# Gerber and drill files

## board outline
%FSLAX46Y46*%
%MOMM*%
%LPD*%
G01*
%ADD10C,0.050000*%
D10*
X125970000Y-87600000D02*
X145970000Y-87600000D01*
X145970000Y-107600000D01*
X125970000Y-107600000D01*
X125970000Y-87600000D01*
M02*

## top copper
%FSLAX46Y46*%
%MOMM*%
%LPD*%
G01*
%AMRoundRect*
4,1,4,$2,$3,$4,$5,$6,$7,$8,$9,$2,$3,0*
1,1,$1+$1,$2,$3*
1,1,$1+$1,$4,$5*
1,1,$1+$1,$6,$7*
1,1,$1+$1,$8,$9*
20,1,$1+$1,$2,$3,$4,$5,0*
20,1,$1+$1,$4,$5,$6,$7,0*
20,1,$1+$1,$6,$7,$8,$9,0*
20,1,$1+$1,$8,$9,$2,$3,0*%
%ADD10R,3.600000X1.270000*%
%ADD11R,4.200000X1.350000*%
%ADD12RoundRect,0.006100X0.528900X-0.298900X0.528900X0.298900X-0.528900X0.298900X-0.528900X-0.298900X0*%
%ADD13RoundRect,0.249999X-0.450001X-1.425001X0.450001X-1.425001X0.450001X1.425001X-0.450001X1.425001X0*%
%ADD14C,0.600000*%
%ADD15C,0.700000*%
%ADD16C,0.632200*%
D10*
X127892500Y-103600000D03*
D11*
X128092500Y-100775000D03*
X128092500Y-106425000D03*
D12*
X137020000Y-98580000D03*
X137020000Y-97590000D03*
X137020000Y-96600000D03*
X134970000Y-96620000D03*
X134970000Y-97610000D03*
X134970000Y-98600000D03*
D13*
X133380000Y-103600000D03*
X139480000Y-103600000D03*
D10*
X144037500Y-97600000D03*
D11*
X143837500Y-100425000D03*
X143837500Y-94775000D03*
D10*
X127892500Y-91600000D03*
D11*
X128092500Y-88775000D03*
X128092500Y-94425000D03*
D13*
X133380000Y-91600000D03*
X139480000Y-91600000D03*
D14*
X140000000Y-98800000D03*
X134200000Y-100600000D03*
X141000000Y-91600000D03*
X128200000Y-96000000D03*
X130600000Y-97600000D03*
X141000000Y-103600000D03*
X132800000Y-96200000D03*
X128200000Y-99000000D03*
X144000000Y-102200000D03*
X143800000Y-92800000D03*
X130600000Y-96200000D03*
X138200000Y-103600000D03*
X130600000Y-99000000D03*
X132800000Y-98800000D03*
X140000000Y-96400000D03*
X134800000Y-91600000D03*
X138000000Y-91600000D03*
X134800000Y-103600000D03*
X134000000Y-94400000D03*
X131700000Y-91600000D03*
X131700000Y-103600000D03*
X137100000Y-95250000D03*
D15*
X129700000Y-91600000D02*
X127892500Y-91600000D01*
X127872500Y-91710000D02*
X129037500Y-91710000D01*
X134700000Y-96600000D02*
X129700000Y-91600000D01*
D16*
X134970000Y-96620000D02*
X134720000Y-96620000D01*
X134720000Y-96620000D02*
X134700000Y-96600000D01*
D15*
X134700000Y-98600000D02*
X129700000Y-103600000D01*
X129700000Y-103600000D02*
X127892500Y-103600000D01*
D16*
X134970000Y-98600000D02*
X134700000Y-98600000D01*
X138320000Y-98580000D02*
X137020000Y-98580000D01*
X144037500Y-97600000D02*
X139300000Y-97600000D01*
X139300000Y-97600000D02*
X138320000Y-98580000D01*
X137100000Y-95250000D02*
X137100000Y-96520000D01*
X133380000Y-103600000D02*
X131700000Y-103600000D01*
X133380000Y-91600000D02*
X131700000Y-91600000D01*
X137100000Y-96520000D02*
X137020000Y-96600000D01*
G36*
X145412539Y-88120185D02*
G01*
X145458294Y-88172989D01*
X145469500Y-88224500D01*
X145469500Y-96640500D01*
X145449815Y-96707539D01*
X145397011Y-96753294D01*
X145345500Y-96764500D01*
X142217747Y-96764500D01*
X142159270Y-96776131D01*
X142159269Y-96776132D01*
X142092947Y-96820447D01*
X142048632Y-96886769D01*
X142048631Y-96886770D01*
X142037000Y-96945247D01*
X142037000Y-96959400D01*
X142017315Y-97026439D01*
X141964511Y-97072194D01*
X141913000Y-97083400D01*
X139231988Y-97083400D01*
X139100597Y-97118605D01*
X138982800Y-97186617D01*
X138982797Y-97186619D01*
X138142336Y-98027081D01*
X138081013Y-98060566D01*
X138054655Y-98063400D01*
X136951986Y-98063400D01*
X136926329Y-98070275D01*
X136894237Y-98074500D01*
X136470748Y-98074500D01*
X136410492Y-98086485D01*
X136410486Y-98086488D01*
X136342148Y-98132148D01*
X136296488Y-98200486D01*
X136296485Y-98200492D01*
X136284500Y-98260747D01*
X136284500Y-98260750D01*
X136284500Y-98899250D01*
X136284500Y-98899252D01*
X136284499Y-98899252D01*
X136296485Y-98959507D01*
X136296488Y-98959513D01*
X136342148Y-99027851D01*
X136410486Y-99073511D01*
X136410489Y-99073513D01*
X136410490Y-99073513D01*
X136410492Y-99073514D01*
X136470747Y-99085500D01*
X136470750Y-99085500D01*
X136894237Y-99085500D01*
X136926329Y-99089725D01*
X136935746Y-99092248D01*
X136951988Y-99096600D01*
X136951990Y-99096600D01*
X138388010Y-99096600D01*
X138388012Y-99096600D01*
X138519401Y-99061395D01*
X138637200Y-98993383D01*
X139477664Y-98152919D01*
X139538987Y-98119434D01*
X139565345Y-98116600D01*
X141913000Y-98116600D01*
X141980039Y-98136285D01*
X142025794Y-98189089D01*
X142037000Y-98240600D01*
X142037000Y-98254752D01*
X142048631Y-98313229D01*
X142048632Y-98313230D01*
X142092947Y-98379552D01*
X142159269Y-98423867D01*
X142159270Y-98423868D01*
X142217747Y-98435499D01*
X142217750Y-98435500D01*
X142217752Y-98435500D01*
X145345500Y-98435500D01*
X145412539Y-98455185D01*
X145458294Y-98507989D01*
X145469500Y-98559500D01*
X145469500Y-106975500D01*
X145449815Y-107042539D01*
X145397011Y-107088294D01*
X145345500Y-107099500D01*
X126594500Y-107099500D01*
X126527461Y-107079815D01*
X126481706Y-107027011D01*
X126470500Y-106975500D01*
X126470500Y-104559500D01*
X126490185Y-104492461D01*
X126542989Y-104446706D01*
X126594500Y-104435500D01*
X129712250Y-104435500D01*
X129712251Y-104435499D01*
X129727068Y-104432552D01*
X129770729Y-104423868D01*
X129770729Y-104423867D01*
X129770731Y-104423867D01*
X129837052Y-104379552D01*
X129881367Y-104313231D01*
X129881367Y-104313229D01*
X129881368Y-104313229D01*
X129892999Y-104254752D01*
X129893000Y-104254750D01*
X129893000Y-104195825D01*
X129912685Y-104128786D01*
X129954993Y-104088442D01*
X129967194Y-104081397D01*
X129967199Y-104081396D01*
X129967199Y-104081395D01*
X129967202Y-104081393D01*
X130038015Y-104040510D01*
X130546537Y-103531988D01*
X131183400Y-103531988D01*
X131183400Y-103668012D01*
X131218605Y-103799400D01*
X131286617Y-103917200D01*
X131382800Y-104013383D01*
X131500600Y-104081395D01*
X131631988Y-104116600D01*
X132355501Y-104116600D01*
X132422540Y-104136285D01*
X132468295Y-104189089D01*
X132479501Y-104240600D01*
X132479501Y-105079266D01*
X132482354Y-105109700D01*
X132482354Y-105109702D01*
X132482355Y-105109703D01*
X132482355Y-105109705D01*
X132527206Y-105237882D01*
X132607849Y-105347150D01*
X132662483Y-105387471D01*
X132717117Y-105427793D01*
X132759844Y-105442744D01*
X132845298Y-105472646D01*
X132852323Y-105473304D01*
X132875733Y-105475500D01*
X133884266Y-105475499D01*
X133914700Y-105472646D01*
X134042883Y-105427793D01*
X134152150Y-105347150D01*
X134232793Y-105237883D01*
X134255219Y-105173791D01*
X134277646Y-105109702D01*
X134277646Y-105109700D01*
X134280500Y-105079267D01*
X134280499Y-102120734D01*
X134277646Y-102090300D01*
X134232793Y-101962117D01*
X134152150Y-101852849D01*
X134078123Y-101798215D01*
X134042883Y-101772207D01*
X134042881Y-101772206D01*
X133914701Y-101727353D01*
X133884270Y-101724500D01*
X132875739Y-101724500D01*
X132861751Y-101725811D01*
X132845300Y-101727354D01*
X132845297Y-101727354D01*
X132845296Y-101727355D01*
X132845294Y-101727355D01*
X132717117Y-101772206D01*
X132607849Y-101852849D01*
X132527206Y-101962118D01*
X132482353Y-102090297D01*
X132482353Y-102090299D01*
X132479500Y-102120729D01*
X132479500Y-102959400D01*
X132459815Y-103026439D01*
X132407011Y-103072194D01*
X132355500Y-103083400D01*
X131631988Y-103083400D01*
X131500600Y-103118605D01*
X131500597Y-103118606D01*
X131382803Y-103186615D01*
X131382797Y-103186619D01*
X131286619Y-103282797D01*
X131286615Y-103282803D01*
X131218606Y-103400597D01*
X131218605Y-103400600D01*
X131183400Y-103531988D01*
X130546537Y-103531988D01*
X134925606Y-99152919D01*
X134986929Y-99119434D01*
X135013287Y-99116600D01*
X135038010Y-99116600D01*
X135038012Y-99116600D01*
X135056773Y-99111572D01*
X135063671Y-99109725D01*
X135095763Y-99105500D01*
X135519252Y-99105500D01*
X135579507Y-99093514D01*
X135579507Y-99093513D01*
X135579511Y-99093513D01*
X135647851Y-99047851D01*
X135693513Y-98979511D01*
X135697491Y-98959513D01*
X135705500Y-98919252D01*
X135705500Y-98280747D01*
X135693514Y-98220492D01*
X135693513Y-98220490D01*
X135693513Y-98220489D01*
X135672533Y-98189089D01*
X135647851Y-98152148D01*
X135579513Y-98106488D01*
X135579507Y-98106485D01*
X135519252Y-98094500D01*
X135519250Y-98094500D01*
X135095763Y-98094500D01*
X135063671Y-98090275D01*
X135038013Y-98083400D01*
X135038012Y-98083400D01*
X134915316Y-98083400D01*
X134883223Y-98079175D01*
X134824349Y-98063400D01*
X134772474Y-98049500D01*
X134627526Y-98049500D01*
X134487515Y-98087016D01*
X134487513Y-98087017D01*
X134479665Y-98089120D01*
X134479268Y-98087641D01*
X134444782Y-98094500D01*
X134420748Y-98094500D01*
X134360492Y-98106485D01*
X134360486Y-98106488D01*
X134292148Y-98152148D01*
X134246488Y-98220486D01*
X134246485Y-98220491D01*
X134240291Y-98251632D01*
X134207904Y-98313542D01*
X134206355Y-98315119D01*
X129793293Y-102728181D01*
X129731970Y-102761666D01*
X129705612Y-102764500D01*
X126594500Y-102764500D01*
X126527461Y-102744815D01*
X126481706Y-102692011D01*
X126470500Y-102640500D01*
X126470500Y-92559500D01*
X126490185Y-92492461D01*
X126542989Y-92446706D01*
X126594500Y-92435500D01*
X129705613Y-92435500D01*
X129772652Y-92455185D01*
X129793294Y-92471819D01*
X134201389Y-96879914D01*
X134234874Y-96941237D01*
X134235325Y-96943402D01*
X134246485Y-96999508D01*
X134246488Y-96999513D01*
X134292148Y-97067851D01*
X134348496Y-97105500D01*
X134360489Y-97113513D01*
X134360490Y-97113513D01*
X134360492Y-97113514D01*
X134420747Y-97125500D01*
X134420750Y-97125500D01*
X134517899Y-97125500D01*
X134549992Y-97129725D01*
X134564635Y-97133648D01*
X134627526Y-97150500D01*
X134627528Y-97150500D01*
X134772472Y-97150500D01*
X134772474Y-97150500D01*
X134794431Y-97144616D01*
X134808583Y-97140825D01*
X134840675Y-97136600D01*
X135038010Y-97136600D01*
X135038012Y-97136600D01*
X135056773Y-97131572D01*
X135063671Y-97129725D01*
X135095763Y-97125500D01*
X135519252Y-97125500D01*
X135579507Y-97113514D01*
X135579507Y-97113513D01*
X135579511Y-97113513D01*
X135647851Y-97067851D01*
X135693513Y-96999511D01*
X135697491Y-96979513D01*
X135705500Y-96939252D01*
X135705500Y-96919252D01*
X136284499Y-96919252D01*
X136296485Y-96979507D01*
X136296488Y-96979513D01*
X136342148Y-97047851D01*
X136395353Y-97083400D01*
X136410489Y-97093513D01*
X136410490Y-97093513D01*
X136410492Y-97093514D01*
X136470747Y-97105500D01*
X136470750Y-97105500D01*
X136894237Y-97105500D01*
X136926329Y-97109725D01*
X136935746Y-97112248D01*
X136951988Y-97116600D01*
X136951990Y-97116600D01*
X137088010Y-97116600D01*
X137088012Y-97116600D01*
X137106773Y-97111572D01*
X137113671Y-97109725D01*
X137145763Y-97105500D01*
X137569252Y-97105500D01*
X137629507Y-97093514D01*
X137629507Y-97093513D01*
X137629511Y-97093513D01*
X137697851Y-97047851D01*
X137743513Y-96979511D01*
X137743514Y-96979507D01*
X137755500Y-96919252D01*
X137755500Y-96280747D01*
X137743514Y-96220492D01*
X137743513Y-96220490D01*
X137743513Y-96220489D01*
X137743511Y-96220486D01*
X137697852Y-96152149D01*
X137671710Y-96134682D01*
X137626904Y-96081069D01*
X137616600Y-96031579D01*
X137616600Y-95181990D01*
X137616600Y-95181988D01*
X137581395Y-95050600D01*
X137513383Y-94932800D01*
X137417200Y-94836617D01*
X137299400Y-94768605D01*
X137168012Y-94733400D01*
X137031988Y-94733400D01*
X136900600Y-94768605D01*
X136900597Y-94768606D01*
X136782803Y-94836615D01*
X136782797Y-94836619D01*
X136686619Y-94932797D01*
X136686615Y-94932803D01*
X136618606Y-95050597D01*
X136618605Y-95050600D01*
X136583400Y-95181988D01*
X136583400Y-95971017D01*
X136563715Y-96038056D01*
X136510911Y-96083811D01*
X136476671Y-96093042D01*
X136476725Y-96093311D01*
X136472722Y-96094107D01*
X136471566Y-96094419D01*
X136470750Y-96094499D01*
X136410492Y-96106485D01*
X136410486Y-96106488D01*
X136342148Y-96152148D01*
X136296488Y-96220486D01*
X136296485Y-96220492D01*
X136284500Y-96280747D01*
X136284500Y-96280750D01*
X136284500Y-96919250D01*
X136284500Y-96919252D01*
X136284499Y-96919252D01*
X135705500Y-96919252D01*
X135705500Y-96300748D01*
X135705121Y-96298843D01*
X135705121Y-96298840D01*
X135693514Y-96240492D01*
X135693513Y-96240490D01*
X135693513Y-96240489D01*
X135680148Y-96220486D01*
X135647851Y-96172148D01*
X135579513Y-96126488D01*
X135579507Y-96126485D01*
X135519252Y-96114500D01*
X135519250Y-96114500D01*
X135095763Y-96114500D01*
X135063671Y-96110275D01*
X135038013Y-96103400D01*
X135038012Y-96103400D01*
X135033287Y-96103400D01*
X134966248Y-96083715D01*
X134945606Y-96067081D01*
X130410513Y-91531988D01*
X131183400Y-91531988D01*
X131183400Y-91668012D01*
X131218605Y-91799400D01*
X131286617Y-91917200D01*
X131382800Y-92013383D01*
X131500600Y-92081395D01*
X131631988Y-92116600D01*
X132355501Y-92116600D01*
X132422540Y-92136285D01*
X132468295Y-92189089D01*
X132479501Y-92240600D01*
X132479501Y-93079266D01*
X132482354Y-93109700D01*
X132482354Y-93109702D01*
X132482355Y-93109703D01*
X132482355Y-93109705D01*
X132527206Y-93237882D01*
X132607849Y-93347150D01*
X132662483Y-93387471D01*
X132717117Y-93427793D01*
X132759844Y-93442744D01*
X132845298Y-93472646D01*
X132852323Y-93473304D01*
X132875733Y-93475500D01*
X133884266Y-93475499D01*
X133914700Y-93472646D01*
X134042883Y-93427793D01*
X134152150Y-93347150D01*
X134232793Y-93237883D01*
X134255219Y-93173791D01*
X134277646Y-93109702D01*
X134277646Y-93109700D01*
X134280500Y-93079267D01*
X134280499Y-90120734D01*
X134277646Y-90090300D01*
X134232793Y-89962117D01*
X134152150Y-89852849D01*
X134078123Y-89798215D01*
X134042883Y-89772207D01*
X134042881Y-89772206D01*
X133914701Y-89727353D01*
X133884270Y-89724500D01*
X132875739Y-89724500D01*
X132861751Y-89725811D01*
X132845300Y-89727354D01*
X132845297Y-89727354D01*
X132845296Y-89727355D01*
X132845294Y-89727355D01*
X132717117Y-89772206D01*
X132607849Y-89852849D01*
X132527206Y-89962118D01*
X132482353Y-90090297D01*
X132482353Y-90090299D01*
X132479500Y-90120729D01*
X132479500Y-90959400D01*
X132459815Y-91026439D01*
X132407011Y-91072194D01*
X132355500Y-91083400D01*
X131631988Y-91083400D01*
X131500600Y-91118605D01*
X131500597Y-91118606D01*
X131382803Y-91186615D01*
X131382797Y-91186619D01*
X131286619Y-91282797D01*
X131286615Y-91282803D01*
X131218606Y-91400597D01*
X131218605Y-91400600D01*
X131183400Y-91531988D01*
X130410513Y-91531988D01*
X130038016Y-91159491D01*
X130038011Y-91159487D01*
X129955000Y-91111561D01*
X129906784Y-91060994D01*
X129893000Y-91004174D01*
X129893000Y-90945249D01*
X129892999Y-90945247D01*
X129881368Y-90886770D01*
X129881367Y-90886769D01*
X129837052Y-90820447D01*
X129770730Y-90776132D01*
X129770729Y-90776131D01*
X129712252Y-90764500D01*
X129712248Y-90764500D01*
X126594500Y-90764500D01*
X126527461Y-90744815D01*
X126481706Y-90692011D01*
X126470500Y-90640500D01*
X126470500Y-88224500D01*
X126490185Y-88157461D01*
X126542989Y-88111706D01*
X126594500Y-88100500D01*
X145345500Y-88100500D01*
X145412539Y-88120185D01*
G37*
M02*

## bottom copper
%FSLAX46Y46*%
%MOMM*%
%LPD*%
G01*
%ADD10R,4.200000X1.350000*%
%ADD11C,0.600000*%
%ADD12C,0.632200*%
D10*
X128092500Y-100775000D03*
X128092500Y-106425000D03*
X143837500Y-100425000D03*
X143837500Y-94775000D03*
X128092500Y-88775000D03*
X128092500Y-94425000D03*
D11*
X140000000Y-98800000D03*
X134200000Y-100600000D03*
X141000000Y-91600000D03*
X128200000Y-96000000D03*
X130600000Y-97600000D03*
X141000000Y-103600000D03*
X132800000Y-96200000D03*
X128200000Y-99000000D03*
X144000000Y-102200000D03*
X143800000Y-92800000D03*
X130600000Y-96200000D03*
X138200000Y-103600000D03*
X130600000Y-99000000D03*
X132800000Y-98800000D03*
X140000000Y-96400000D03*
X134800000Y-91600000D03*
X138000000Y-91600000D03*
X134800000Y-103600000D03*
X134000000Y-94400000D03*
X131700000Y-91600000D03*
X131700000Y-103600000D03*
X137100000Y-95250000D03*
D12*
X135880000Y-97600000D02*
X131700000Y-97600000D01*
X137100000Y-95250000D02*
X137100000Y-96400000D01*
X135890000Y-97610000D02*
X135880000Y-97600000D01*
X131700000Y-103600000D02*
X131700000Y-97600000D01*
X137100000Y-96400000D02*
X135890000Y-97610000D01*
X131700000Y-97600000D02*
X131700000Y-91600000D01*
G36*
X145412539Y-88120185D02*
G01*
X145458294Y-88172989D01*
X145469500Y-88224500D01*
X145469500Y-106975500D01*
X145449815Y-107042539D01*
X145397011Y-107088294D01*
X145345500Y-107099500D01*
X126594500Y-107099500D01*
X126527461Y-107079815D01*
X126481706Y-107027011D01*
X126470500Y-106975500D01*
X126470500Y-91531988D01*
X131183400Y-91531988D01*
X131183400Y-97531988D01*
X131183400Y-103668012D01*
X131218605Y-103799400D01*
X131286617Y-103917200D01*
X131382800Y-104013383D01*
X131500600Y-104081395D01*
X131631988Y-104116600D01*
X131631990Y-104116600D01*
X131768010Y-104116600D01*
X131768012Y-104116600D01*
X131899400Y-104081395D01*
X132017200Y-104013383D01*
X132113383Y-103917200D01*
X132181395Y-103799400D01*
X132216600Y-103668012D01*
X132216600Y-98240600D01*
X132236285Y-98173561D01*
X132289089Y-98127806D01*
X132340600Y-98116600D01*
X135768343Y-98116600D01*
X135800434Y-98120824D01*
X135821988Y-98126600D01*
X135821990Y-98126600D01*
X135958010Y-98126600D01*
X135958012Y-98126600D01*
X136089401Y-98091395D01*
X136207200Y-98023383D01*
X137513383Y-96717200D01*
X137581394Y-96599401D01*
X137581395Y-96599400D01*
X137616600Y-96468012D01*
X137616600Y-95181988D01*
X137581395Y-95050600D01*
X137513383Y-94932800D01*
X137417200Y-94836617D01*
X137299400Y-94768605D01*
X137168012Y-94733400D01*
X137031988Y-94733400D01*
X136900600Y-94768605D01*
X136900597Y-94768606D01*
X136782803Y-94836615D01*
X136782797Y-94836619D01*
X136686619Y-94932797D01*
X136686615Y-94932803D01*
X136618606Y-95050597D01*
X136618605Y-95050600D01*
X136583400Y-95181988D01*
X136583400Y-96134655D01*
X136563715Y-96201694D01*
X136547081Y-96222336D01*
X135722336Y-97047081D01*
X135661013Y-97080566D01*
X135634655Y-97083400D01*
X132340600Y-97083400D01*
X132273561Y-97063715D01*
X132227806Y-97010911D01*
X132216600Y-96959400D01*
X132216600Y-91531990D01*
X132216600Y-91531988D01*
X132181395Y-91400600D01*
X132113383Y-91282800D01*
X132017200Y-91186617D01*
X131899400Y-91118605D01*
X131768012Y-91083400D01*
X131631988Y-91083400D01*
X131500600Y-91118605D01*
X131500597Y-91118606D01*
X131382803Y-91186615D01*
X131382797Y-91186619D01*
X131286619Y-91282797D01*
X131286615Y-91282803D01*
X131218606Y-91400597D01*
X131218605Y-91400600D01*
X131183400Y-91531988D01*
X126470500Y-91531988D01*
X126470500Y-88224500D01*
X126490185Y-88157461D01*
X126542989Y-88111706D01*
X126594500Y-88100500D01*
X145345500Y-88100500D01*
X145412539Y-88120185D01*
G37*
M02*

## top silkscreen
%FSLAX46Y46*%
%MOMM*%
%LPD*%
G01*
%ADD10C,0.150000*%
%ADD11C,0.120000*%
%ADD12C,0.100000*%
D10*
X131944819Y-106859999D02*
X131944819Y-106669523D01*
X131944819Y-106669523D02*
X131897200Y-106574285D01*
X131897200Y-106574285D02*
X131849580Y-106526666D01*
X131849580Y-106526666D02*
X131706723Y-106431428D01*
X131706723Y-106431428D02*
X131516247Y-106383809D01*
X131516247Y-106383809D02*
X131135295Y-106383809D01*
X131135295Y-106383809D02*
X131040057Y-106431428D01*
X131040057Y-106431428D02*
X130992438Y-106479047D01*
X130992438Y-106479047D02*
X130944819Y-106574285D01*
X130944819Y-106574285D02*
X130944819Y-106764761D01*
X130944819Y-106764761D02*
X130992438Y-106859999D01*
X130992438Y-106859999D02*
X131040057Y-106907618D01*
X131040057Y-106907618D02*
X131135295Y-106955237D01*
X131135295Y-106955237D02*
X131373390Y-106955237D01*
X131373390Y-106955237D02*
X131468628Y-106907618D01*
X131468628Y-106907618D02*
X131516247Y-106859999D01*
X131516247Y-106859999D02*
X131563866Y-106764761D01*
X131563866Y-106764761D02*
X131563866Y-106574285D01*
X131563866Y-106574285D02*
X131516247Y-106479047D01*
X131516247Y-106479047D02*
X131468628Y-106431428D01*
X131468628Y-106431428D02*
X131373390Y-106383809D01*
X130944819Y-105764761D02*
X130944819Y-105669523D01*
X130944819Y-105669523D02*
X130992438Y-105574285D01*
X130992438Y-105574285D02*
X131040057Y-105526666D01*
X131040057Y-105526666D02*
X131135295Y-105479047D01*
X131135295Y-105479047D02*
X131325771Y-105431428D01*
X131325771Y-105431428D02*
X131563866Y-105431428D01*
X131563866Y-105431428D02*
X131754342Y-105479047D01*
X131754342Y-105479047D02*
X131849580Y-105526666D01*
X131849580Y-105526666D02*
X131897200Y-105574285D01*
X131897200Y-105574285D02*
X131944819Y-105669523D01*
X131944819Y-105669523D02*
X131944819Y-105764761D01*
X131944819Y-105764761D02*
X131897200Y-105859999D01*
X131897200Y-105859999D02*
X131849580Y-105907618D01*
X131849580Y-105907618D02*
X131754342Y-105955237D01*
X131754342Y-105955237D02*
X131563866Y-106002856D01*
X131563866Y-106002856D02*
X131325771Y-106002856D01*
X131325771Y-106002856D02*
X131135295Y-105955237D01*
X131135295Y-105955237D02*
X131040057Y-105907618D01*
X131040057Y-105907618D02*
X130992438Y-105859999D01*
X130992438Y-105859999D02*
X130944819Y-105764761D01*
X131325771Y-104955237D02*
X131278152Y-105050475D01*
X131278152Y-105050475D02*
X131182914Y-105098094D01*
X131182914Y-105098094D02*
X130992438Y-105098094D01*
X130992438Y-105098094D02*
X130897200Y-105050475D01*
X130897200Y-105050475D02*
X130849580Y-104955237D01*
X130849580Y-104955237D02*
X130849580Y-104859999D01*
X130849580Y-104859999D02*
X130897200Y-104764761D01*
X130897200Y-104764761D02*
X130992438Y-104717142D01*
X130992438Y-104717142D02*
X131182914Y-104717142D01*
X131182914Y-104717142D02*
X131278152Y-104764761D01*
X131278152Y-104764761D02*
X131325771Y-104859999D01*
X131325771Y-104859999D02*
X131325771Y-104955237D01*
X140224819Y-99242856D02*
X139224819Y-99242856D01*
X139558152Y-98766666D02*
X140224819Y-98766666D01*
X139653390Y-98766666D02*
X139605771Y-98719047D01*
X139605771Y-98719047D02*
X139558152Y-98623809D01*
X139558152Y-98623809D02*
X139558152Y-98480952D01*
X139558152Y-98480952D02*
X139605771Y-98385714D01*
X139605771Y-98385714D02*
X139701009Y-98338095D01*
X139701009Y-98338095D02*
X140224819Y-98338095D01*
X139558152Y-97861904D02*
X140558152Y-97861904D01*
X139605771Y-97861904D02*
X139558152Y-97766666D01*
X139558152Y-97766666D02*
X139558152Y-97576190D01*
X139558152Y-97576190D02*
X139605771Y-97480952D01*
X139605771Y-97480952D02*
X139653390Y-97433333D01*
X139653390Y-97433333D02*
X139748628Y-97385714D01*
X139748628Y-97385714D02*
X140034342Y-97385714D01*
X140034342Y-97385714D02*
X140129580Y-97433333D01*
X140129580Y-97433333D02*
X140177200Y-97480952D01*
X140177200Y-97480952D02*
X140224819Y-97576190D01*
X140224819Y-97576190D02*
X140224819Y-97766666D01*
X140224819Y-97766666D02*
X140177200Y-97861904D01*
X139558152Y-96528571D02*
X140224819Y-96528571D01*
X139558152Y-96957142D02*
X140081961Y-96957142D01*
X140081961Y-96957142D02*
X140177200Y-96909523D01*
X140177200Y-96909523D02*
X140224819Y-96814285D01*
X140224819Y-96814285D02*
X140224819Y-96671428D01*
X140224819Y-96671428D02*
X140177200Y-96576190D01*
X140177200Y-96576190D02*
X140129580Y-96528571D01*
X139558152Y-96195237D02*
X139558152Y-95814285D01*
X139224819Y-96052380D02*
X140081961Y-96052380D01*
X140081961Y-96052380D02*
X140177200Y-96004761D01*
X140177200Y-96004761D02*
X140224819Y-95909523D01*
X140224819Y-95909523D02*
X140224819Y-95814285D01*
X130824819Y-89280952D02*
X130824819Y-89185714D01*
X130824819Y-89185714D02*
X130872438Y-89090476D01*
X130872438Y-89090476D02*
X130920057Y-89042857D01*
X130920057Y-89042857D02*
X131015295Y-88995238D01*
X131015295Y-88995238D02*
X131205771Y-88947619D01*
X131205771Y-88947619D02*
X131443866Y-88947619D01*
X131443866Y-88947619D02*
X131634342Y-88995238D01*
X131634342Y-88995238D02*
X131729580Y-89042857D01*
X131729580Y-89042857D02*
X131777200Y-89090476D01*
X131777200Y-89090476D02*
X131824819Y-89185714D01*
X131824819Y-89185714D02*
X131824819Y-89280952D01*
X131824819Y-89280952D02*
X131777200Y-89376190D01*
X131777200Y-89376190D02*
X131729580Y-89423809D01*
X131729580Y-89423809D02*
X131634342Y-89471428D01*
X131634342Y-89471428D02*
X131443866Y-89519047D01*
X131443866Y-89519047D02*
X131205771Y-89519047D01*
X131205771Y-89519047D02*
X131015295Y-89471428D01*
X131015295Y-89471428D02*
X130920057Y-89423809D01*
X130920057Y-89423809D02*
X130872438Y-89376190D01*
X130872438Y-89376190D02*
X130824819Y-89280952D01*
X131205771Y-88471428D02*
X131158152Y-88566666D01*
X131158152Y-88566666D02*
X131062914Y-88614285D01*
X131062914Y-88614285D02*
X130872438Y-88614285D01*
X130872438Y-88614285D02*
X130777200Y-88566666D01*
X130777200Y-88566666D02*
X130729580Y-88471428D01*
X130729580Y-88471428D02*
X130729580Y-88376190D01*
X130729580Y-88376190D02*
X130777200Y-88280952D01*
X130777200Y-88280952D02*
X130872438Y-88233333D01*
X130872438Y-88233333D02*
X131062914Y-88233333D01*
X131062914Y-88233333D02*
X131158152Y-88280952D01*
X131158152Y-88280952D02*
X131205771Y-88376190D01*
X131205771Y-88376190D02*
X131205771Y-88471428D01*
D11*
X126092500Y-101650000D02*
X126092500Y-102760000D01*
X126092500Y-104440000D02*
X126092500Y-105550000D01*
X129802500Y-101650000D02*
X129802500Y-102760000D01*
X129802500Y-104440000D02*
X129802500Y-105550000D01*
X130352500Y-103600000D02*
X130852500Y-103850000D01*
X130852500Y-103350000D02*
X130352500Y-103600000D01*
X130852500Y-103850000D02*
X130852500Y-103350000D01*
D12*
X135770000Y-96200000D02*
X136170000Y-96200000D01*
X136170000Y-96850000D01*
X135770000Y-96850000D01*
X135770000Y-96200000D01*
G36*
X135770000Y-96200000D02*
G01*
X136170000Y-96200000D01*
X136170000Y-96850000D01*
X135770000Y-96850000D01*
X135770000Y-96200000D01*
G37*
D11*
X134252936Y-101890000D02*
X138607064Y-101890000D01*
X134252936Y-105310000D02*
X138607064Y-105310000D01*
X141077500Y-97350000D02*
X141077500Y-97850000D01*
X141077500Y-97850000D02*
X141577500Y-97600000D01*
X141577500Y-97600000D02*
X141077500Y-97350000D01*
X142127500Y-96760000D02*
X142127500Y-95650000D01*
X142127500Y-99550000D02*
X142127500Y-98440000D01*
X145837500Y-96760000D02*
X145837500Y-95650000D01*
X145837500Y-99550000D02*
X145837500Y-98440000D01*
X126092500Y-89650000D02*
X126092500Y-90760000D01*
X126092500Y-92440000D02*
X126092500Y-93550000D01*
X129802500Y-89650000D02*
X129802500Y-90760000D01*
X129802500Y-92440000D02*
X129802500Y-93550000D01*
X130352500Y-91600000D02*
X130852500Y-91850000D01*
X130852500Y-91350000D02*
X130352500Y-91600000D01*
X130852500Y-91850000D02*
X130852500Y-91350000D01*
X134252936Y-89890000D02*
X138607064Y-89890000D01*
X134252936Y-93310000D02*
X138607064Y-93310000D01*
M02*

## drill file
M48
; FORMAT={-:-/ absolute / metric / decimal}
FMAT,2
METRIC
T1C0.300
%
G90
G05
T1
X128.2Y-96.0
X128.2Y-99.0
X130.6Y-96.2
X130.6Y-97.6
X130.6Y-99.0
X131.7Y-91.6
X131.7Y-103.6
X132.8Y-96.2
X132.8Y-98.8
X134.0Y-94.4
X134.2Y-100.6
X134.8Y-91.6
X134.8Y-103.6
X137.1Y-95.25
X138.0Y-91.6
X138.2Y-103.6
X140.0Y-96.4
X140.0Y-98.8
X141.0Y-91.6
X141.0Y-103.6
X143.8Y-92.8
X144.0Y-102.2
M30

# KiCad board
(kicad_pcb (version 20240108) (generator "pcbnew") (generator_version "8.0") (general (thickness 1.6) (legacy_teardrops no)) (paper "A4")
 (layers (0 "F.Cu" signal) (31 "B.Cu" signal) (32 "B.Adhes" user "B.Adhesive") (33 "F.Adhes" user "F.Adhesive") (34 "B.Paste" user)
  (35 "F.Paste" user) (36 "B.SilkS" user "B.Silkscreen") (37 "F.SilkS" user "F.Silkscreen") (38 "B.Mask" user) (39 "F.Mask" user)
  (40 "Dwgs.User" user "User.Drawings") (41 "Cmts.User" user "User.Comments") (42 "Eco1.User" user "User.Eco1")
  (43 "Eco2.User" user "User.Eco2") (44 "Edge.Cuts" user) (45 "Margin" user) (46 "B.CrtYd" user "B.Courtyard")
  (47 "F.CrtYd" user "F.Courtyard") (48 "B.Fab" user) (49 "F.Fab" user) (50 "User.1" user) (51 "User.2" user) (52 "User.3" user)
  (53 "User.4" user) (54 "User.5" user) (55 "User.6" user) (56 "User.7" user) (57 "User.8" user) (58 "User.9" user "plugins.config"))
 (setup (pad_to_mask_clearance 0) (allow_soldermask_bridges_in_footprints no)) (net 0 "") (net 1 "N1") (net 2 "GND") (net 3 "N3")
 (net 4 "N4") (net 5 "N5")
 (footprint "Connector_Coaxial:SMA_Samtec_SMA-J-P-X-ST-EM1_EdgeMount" (layer "F.Cu") (at 128.0925 103.6 -90)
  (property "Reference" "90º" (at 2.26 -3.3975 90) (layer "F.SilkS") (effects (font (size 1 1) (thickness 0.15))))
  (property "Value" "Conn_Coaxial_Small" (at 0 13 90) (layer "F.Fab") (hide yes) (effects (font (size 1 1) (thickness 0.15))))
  (fp_line (start -1.95 2) (end -0.84 2) (stroke (width 0.12) (type solid)) (layer "F.SilkS"))
  (fp_line (start 0.84 2) (end 1.95 2) (stroke (width 0.12) (type solid)) (layer "F.SilkS"))
  (fp_line (start -1.95 -1.71) (end -0.84 -1.71) (stroke (width 0.12) (type solid)) (layer "F.SilkS"))
  (fp_line (start 0.84 -1.71) (end 1.95 -1.71) (stroke (width 0.12) (type solid)) (layer "F.SilkS"))
  (fp_line (start 0 -2.26) (end 0.25 -2.76) (stroke (width 0.12) (type solid)) (layer "F.SilkS"))
  (fp_line (start -0.25 -2.76) (end 0 -2.26) (stroke (width 0.12) (type solid)) (layer "F.SilkS"))
  (fp_line (start 0.25 -2.76) (end -0.25 -2.76) (stroke (width 0.12) (type solid)) (layer "F.SilkS"))
  (pad "1" smd rect (at 0 0.2 270) (size 1.27 3.6) (layers "F.Cu" "F.Paste" "F.Mask") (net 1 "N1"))
  (pad "2" smd rect (at -2.825 0 270) (size 1.35 4.2) (layers "F.Cu" "F.Paste" "F.Mask") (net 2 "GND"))
  (pad "2" smd rect (at -2.825 0 270) (size 1.35 4.2) (layers "B.Cu" "B.Paste" "B.Mask") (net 2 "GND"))
  (pad "2" smd rect (at 2.825 0 270) (size 1.35 4.2) (layers "F.Cu" "F.Paste" "F.Mask") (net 2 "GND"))
  (pad "2" smd rect (at 2.825 0 270) (size 1.35 4.2) (layers "B.Cu" "B.Paste" "B.Mask") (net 2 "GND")))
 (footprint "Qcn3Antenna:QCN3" (layer "F.Cu") (at 136.97 97.6 90)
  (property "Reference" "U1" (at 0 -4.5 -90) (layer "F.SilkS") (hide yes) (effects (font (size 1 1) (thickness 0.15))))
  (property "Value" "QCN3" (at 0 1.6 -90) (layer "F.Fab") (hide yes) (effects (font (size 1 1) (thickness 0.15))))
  (fp_rect (start 0.75 -1.2) (end 1.4 -0.8) (stroke (width 0.1) (type solid)) (fill solid) (layer "F.SilkS"))
  (pad "1" smd roundrect (at -0.98 0.05 90) (size 0.61 1.07) (layers "F.Cu" "F.Paste" "F.Mask") (roundrect_rratio 0.01) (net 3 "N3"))
  (pad "2" smd roundrect (at 0.01 0.05 90) (size 0.61 1.07) (layers "F.Cu" "F.Paste" "F.Mask") (roundrect_rratio 0.01) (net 2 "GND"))
  (pad "3" smd roundrect (at 1 0.05 90) (size 0.61 1.07) (layers "F.Cu" "F.Paste" "F.Mask") (roundrect_rratio 0.01) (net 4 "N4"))
  (pad "4" smd roundrect (at 0.98 -2 90) (size 0.61 1.07) (layers "F.Cu" "F.Paste" "F.Mask") (roundrect_rratio 0.01) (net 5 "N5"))
  (pad "5" smd roundrect (at -0.01 -2 90) (size 0.61 1.07) (layers "F.Cu" "F.Paste" "F.Mask") (roundrect_rratio 0.01) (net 2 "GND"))
  (pad "6" smd roundrect (at -1 -2 90) (size 0.61 1.07) (layers "F.Cu" "F.Paste" "F.Mask") (roundrect_rratio 0.01) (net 1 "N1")))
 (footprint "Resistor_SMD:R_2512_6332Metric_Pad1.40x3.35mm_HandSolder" (layer "F.Cu") (at 136.43 103.6)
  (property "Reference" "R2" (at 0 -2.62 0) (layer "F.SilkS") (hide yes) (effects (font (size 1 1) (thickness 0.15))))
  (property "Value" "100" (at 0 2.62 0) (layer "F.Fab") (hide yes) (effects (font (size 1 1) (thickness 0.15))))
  (fp_line (start -2.177064 -1.71) (end 2.177064 -1.71) (stroke (width 0.12) (type solid)) (layer "F.SilkS"))
  (fp_line (start -2.177064 1.71) (end 2.177064 1.71) (stroke (width 0.12) (type solid)) (layer "F.SilkS"))
  (pad "1" smd roundrect (at -3.05 0) (size 1.4 3.35) (layers "F.Cu" "F.Paste" "F.Mask") (roundrect_rratio 0.178571) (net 4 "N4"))
  (pad "2" smd roundrect (at 3.05 0) (size 1.4 3.35) (layers "F.Cu" "F.Paste" "F.Mask") (roundrect_rratio 0.178571) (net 2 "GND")))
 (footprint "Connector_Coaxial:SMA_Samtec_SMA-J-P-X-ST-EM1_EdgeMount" (layer "F.Cu") (at 143.8375 97.6 90)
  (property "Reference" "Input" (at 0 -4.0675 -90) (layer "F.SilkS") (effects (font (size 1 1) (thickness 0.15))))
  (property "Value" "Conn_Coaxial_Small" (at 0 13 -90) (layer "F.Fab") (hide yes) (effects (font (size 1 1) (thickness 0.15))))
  (fp_line (start 0.25 -2.76) (end -0.25 -2.76) (stroke (width 0.12) (type solid)) (layer "F.SilkS"))
  (fp_line (start -0.25 -2.76) (end 0 -2.26) (stroke (width 0.12) (type solid)) (layer "F.SilkS"))
  (fp_line (start 0 -2.26) (end 0.25 -2.76) (stroke (width 0.12) (type solid)) (layer "F.SilkS"))
  (fp_line (start 0.84 -1.71) (end 1.95 -1.71) (stroke (width 0.12) (type solid)) (layer "F.SilkS"))
  (fp_line (start -1.95 -1.71) (end -0.84 -1.71) (stroke (width 0.12) (type solid)) (layer "F.SilkS"))
  (fp_line (start 0.84 2) (end 1.95 2) (stroke (width 0.12) (type solid)) (layer "F.SilkS"))
  (fp_line (start -1.95 2) (end -0.84 2) (stroke (width 0.12) (type solid)) (layer "F.SilkS"))
  (pad "1" smd rect (at 0 0.2 90) (size 1.27 3.6) (layers "F.Cu" "F.Paste" "F.Mask") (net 3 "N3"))
  (pad "2" smd rect (at -2.825 0 90) (size 1.35 4.2) (layers "F.Cu" "F.Paste" "F.Mask") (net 2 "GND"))
  (pad "2" smd rect (at -2.825 0 90) (size 1.35 4.2) (layers "B.Cu" "B.Paste" "B.Mask") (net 2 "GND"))
  (pad "2" smd rect (at 2.825 0 90) (size 1.35 4.2) (layers "F.Cu" "F.Paste" "F.Mask") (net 2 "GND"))
  (pad "2" smd rect (at 2.825 0 90) (size 1.35 4.2) (layers "B.Cu" "B.Paste" "B.Mask") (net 2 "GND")))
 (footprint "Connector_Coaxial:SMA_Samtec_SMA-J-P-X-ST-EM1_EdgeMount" (layer "F.Cu") (at 128.0925 91.6 -90)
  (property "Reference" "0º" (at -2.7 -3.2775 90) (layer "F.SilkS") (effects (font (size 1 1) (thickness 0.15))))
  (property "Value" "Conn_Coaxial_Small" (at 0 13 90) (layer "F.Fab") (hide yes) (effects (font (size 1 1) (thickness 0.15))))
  (fp_line (start -1.95 2) (end -0.84 2) (stroke (width 0.12) (type solid)) (layer "F.SilkS"))
  (fp_line (start 0.84 2) (end 1.95 2) (stroke (width 0.12) (type solid)) (layer "F.SilkS"))
  (fp_line (start -1.95 -1.71) (end -0.84 -1.71) (stroke (width 0.12) (type solid)) (layer "F.SilkS"))
  (fp_line (start 0.84 -1.71) (end 1.95 -1.71) (stroke (width 0.12) (type solid)) (layer "F.SilkS"))
  (fp_line (start 0 -2.26) (end 0.25 -2.76) (stroke (width 0.12) (type solid)) (layer "F.SilkS"))
  (fp_line (start -0.25 -2.76) (end 0 -2.26) (stroke (width 0.12) (type solid)) (layer "F.SilkS"))
  (fp_line (start 0.25 -2.76) (end -0.25 -2.76) (stroke (width 0.12) (type solid)) (layer "F.SilkS"))
  (pad "1" smd rect (at 0 0.2 270) (size 1.27 3.6) (layers "F.Cu" "F.Paste" "F.Mask") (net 5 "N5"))
  (pad "2" smd rect (at -2.825 0 270) (size 1.35 4.2) (layers "F.Cu" "F.Paste" "F.Mask") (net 2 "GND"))
  (pad "2" smd rect (at -2.825 0 270) (size 1.35 4.2) (layers "B.Cu" "B.Paste" "B.Mask") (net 2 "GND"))
  (pad "2" smd rect (at 2.825 0 270) (size 1.35 4.2) (layers "F.Cu" "F.Paste" "F.Mask") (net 2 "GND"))
  (pad "2" smd rect (at 2.825 0 270) (size 1.35 4.2) (layers "B.Cu" "B.Paste" "B.Mask") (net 2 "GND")))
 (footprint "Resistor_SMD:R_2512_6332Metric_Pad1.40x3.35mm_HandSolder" (layer "F.Cu") (at 136.43 91.6)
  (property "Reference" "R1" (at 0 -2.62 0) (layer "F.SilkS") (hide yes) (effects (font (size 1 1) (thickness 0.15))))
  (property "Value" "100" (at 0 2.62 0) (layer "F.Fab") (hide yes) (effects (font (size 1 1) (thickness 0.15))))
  (fp_line (start -2.177064 -1.71) (end 2.177064 -1.71) (stroke (width 0.12) (type solid)) (layer "F.SilkS"))
  (fp_line (start -2.177064 1.71) (end 2.177064 1.71) (stroke (width 0.12) (type solid)) (layer "F.SilkS"))
  (pad "1" smd roundrect (at -3.05 0) (size 1.4 3.35) (layers "F.Cu" "F.Paste" "F.Mask") (roundrect_rratio 0.178571) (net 4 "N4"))
  (pad "2" smd roundrect (at 3.05 0) (size 1.4 3.35) (layers "F.Cu" "F.Paste" "F.Mask") (roundrect_rratio 0.178571) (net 2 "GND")))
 (gr_rect (start 125.97 87.6) (end 145.97 107.6) (stroke (width 0.05) (type default)) (fill none) (layer "Edge.Cuts"))
 (via (at 140 98.8) (size 0.6) (drill 0.3) (layers "F.Cu" "B.Cu") (free yes) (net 2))
 (via (at 134.2 100.6) (size 0.6) (drill 0.3) (layers "F.Cu" "B.Cu") (free yes) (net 2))
 (via (at 141 91.6) (size 0.6) (drill 0.3) (layers "F.Cu" "B.Cu") (free yes) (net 2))
 (via (at 128.2 96) (size 0.6) (drill 0.3) (layers "F.Cu" "B.Cu") (free yes) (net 2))
 (via (at 130.6 97.6) (size 0.6) (drill 0.3) (layers "F.Cu" "B.Cu") (free yes) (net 2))
 (via (at 141 103.6) (size 0.6) (drill 0.3) (layers "F.Cu" "B.Cu") (free yes) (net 2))
 (via (at 132.8 96.2) (size 0.6) (drill 0.3) (layers "F.Cu" "B.Cu") (free yes) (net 2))
 (via (at 128.2 99) (size 0.6) (drill 0.3) (layers "F.Cu" "B.Cu") (free yes) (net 2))
 (via (at 144 102.2) (size 0.6) (drill 0.3) (layers "F.Cu" "B.Cu") (free yes) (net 2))
 (via (at 143.8 92.8) (size 0.6) (drill 0.3) (layers "F.Cu" "B.Cu") (free yes) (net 2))
 (via (at 130.6 96.2) (size 0.6) (drill 0.3) (layers "F.Cu" "B.Cu") (free yes) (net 2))
 (via (at 138.2 103.6) (size 0.6) (drill 0.3) (layers "F.Cu" "B.Cu") (free yes) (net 2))
 (via (at 130.6 99) (size 0.6) (drill 0.3) (layers "F.Cu" "B.Cu") (free yes) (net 2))
 (via (at 132.8 98.8) (size 0.6) (drill 0.3) (layers "F.Cu" "B.Cu") (free yes) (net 2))
 (via (at 140 96.4) (size 0.6) (drill 0.3) (layers "F.Cu" "B.Cu") (free yes) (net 2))
 (via (at 134.8 91.6) (size 0.6) (drill 0.3) (layers "F.Cu" "B.Cu") (free yes) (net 2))
 (via (at 138 91.6) (size 0.6) (drill 0.3) (layers "F.Cu" "B.Cu") (free yes) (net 2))
 (via (at 134.8 103.6) (size 0.6) (drill 0.3) (layers "F.Cu" "B.Cu") (free yes) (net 2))
 (via (at 134 94.4) (size 0.6) (drill 0.3) (layers "F.Cu" "B.Cu") (free yes) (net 2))
 (segment (start 129.7 91.6) (end 127.8925 91.6) (width 0.7) (layer "F.Cu") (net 5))
 (segment (start 127.8725 91.71) (end 129.0375 91.71) (width 0.7) (layer "F.Cu") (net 5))
 (segment (start 134.7 96.6) (end 129.7 91.6) (width 0.7) (layer "F.Cu") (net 5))
 (segment (start 134.97 96.62) (end 134.72 96.62) (width 0.6322) (layer "F.Cu") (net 5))
 (segment (start 134.72 96.62) (end 134.7 96.6) (width 0.6322) (layer "F.Cu") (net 5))
 (segment (start 134.7 98.6) (end 129.7 103.6) (width 0.7) (layer "F.Cu") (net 1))
 (segment (start 129.7 103.6) (end 127.8925 103.6) (width 0.7) (layer "F.Cu") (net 1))
 (segment (start 134.97 98.6) (end 134.7 98.6) (width 0.6322) (layer "F.Cu") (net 1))
 (segment (start 138.32 98.58) (end 137.02 98.58) (width 0.6322) (layer "F.Cu") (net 3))
 (segment (start 144.0375 97.6) (end 139.3 97.6) (width 0.6322) (layer "F.Cu") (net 3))
 (segment (start 139.3 97.6) (end 138.32 98.58) (width 0.6322) (layer "F.Cu") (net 3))
 (segment (start 137.1 95.25) (end 137.1 96.52) (width 0.6322) (layer "F.Cu") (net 4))
 (segment (start 133.38 103.6) (end 131.7 103.6) (width 0.6322) (layer "F.Cu") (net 4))
 (segment (start 133.38 91.6) (end 131.7 91.6) (width 0.6322) (layer "F.Cu") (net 4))
 (segment (start 137.1 96.52) (end 137.02 96.6) (width 0.6322) (layer "F.Cu") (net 4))
 (via (at 131.7 91.6) (size 0.6) (drill 0.3) (layers "F.Cu" "B.Cu") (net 4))
 (via (at 131.7 103.6) (size 0.6) (drill 0.3) (layers "F.Cu" "B.Cu") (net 4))
 (via (at 137.1 95.25) (size 0.6) (drill 0.3) (layers "F.Cu" "B.Cu") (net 4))
 (segment (start 135.88 97.6) (end 131.7 97.6) (width 0.6322) (layer "B.Cu") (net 4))
 (segment (start 137.1 95.25) (end 137.1 96.4) (width 0.6322) (layer "B.Cu") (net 4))
 (segment (start 135.89 97.61) (end 135.88 97.6) (width 0.6322) (layer "B.Cu") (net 4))
 (segment (start 131.7 103.6) (end 131.7 97.6) (width 0.6322) (layer "B.Cu") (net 4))
 (segment (start 137.1 96.4) (end 135.89 97.61) (width 0.6322) (layer "B.Cu") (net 4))
 (segment (start 131.7 97.6) (end 131.7 91.6) (width 0.6322) (layer "B.Cu") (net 4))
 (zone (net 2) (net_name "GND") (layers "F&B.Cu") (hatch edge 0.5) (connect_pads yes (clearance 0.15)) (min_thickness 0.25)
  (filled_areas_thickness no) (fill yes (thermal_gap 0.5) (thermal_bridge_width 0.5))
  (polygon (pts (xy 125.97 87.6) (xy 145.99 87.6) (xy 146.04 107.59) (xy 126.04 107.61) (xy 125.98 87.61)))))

